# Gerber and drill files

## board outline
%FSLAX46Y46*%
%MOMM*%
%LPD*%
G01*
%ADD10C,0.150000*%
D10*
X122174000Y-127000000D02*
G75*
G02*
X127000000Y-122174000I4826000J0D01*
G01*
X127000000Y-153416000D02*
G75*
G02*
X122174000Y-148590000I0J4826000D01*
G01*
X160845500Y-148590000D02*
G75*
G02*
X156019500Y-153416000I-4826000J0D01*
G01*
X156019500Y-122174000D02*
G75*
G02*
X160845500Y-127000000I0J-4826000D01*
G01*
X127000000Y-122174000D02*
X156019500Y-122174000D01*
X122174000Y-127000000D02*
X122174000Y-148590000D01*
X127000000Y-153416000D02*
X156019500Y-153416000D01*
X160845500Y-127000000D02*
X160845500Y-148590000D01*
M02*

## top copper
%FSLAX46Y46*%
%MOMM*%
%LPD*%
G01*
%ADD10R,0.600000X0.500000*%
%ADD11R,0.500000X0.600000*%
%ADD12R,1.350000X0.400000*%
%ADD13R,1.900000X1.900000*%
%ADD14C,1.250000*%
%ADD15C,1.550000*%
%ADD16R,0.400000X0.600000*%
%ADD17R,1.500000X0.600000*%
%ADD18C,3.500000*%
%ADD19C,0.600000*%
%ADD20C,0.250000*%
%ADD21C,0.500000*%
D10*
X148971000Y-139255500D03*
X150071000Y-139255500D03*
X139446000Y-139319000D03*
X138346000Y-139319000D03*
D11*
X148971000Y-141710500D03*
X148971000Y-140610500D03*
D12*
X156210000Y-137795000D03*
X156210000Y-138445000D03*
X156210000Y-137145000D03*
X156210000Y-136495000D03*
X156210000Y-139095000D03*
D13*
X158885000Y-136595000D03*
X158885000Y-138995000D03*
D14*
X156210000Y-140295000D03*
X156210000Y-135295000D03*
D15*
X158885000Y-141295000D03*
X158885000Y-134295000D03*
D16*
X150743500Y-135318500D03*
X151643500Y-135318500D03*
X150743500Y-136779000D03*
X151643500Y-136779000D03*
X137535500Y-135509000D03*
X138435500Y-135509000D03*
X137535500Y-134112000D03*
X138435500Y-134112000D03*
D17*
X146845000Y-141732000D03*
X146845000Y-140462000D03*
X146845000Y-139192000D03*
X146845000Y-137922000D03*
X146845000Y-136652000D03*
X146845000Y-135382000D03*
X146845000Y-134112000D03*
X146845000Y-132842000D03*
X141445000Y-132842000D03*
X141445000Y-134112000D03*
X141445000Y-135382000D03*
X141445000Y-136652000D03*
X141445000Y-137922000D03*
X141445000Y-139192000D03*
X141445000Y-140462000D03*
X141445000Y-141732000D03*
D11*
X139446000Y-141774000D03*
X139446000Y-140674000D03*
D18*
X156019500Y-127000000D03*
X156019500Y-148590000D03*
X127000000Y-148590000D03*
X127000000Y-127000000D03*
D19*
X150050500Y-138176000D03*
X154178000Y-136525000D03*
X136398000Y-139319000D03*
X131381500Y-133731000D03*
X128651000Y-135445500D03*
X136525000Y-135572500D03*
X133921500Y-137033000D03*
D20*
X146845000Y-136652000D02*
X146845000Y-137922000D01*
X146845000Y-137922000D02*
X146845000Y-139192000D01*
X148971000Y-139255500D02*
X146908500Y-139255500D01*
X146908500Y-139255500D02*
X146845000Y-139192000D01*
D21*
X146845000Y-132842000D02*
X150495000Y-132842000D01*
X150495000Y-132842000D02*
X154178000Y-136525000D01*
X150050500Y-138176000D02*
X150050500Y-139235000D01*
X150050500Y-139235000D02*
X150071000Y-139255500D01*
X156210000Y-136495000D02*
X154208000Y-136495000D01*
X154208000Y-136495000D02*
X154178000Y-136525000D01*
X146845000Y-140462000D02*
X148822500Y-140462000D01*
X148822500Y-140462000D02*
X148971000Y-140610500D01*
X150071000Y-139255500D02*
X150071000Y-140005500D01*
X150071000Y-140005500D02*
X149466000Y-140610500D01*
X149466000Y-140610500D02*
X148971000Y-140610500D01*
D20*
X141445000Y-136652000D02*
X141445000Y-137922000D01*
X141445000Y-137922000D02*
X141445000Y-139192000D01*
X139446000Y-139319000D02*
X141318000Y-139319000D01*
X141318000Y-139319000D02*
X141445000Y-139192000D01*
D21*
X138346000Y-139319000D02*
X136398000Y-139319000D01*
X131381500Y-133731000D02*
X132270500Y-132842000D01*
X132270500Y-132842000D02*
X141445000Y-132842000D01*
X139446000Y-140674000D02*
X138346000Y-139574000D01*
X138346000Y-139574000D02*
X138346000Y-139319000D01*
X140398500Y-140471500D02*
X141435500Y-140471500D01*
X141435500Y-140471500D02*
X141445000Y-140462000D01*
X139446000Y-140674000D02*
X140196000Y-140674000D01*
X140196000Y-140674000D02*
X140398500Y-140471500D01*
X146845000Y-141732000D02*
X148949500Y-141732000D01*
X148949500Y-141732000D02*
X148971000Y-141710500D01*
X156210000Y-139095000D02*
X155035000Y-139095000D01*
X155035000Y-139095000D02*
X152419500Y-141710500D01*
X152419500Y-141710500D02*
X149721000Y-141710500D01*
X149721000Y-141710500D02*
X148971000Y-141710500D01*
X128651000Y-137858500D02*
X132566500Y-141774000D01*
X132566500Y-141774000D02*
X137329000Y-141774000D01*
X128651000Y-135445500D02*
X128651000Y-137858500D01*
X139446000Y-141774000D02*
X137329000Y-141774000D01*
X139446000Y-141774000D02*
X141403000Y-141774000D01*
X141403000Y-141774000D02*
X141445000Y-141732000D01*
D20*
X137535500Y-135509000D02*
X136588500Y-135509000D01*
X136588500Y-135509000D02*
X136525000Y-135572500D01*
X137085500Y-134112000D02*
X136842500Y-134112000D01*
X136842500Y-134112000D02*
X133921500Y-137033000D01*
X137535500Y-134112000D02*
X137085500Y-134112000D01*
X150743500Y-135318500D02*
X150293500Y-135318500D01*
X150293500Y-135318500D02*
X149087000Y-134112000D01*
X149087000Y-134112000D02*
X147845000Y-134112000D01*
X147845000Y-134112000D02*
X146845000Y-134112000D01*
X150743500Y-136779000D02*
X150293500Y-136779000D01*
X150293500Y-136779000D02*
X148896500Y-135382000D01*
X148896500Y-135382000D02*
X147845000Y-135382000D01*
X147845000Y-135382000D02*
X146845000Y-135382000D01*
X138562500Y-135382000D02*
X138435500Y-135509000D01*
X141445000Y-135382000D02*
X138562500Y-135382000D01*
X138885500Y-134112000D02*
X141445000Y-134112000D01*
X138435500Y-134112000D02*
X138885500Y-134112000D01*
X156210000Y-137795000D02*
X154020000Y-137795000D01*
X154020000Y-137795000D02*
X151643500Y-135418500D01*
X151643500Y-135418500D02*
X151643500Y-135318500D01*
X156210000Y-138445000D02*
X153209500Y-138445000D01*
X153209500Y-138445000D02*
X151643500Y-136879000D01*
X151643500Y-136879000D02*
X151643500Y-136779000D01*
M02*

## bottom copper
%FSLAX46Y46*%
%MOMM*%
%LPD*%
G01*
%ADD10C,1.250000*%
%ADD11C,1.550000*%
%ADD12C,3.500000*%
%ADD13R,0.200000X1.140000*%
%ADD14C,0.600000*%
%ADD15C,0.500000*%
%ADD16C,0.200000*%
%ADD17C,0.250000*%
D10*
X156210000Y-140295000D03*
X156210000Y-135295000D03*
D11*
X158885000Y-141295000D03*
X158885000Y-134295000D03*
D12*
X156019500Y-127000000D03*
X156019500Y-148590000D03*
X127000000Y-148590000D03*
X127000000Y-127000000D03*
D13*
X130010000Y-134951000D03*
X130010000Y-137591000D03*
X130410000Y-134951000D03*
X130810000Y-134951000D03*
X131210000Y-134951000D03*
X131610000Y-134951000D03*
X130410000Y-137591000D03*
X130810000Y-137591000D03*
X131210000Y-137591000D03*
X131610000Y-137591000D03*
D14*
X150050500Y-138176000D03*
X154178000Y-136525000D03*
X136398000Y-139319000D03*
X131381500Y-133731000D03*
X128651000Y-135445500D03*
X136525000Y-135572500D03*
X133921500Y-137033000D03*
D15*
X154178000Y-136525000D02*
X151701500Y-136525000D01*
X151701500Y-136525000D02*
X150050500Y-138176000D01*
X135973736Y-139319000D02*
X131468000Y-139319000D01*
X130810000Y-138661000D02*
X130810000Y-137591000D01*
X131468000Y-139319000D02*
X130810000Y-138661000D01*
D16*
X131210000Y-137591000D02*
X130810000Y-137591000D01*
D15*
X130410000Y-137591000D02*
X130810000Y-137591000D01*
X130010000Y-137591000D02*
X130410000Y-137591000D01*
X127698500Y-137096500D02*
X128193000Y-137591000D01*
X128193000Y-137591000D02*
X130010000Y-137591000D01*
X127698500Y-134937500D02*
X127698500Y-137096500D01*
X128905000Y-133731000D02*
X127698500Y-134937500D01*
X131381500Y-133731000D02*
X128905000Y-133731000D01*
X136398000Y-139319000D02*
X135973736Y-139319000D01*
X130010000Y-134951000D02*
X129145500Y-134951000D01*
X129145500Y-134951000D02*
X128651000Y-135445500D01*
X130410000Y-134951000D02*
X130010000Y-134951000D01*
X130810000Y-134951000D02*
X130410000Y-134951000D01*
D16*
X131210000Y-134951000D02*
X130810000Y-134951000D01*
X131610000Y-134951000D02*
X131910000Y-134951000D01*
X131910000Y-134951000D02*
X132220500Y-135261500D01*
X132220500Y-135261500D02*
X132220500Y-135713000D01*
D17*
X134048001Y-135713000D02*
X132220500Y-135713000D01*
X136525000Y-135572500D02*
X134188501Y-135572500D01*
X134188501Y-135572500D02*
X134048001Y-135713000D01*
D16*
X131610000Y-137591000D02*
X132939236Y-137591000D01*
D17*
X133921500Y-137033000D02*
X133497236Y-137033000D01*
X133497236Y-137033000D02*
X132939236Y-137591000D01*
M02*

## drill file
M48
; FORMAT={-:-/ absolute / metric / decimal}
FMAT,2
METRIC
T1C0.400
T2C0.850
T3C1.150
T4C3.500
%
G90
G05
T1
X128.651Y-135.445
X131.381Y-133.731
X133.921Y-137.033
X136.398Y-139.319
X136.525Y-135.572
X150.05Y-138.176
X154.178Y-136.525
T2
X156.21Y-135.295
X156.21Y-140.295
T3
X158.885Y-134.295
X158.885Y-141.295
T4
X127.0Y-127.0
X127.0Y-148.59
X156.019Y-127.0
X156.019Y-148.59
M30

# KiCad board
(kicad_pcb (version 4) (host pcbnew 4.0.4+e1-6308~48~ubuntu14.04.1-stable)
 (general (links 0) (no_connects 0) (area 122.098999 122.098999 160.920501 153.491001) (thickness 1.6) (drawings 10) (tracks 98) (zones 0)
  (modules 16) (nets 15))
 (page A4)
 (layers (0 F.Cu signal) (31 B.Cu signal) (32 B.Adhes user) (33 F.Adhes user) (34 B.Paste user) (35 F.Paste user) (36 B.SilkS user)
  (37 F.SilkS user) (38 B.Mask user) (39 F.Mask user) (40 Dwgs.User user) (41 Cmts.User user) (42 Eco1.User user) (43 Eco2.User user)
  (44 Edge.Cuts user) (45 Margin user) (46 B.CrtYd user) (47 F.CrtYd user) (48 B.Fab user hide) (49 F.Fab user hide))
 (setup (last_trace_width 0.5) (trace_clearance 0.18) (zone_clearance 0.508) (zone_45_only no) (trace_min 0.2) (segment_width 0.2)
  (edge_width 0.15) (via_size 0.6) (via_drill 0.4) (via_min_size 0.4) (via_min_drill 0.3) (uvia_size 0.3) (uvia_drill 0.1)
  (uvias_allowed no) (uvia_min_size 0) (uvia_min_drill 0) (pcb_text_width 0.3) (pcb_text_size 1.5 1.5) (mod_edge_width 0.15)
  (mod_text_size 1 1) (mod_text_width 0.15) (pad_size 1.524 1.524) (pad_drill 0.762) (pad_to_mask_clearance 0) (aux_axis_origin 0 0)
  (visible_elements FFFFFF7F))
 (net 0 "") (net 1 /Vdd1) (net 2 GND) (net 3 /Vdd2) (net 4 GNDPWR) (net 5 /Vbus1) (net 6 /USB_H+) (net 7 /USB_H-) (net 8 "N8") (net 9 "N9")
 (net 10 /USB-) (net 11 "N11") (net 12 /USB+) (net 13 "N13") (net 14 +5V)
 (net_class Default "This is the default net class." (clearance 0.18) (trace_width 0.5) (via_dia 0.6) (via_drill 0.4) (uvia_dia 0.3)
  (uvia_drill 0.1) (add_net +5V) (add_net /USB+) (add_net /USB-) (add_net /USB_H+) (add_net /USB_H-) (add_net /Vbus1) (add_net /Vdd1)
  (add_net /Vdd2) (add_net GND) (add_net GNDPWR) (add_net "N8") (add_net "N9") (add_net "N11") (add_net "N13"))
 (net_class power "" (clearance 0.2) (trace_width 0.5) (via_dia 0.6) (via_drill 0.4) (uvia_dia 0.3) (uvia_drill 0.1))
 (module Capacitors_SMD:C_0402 (layer F.Cu) (at 149.521 139.2555)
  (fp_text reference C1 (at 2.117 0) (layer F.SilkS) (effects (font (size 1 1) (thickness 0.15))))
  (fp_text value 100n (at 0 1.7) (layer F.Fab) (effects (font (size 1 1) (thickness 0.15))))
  (pad 1 smd rect (at -0.55 0) (size 0.6 0.5) (layers F.Cu F.Paste F.Mask) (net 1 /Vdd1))
  (pad 2 smd rect (at 0.55 0) (size 0.6 0.5) (layers F.Cu F.Paste F.Mask) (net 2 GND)))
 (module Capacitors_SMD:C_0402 (layer F.Cu) (at 138.896 139.319 180)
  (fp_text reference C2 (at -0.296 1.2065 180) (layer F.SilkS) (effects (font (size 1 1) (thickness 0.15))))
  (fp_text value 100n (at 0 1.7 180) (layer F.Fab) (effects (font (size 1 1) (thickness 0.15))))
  (pad 1 smd rect (at -0.55 0 180) (size 0.6 0.5) (layers F.Cu F.Paste F.Mask) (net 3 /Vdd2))
  (pad 2 smd rect (at 0.55 0 180) (size 0.6 0.5) (layers F.Cu F.Paste F.Mask) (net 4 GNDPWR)))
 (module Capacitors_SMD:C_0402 (layer F.Cu) (at 148.971 141.1605 90)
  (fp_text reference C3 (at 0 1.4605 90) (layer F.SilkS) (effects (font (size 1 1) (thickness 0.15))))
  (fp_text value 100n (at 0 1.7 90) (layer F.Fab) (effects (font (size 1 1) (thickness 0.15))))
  (pad 1 smd rect (at -0.55 0 90) (size 0.6 0.5) (layers F.Cu F.Paste F.Mask) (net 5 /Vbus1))
  (pad 2 smd rect (at 0.55 0 90) (size 0.6 0.5) (layers F.Cu F.Paste F.Mask) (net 2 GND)))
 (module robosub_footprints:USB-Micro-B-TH (layer F.Cu) (at 155.535 137.795 90)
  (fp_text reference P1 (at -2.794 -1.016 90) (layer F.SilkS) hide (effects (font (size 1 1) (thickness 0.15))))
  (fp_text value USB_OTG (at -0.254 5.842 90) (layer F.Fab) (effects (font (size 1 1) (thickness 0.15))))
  (pad 3 smd rect (at 0 0.675 90) (size 0.4 1.35) (layers F.Cu F.Paste F.Mask) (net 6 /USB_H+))
  (pad 2 smd rect (at -0.65 0.675 90) (size 0.4 1.35) (layers F.Cu F.Paste F.Mask) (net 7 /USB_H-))
  (pad 4 smd rect (at 0.65 0.675 90) (size 0.4 1.35) (layers F.Cu F.Paste F.Mask))
  (pad 5 smd rect (at 1.3 0.675 90) (size 0.4 1.35) (layers F.Cu F.Paste F.Mask) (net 2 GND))
  (pad 1 smd rect (at -1.3 0.675 90) (size 0.4 1.35) (layers F.Cu F.Paste F.Mask) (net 5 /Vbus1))
  (pad "" smd rect (at 1.2 3.35 90) (size 1.9 1.9) (layers F.Cu F.Paste F.Mask))
  (pad "" smd rect (at -1.2 3.35 90) (size 1.9 1.9) (layers F.Cu F.Paste F.Mask))
  (pad "" thru_hole circle (at -2.5 0.675 90) (size 1.25 1.25) (drill 0.85) (layers *.Cu *.Mask F.SilkS))
  (pad "" thru_hole circle (at 2.5 0.675 90) (size 1.25 1.25) (drill 0.85) (layers *.Cu *.Mask F.SilkS))
  (pad "" thru_hole circle (at -3.5 3.35 90) (size 1.55 1.55) (drill 1.15) (layers *.Cu *.Mask F.SilkS))
  (pad "" thru_hole circle (at 3.5 3.35 90) (size 1.55 1.55) (drill 1.15) (layers *.Cu *.Mask F.SilkS)))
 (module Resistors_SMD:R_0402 (layer F.Cu) (at 151.1935 135.3185)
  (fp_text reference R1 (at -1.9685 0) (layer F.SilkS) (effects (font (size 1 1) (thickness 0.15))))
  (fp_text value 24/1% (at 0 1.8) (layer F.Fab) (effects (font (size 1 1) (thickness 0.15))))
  (pad 1 smd rect (at -0.45 0) (size 0.4 0.6) (layers F.Cu F.Paste F.Mask) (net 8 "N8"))
  (pad 2 smd rect (at 0.45 0) (size 0.4 0.6) (layers F.Cu F.Paste F.Mask) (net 6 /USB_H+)))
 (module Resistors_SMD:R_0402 (layer F.Cu) (at 151.1935 136.779)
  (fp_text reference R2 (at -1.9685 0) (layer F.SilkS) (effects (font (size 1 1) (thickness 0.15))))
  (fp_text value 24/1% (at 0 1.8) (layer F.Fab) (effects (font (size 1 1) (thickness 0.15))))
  (pad 1 smd rect (at -0.45 0) (size 0.4 0.6) (layers F.Cu F.Paste F.Mask) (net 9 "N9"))
  (pad 2 smd rect (at 0.45 0) (size 0.4 0.6) (layers F.Cu F.Paste F.Mask) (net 7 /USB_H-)))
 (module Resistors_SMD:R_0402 (layer F.Cu) (at 137.9855 135.509)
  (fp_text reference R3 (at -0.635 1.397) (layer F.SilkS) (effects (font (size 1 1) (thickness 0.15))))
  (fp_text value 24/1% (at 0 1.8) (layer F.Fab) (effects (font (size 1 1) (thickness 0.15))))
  (pad 1 smd rect (at -0.45 0) (size 0.4 0.6) (layers F.Cu F.Paste F.Mask) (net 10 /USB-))
  (pad 2 smd rect (at 0.45 0) (size 0.4 0.6) (layers F.Cu F.Paste F.Mask) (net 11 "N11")))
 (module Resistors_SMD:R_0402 (layer F.Cu) (at 137.9855 134.112)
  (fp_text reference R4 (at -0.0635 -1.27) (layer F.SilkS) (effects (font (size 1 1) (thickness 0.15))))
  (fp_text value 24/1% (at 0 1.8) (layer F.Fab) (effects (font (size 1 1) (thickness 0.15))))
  (pad 1 smd rect (at -0.45 0) (size 0.4 0.6) (layers F.Cu F.Paste F.Mask) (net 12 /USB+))
  (pad 2 smd rect (at 0.45 0) (size 0.4 0.6) (layers F.Cu F.Paste F.Mask) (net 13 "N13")))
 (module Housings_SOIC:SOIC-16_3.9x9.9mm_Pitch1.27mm (layer F.Cu) (at 144.145 137.287 180)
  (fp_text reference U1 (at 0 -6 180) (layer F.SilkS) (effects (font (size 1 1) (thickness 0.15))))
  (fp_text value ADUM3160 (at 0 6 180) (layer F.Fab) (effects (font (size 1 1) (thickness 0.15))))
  (pad 1 smd rect (at -2.7 -4.445 180) (size 1.5 0.6) (layers F.Cu F.Paste F.Mask) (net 5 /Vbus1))
  (pad 2 smd rect (at -2.7 -3.175 180) (size 1.5 0.6) (layers F.Cu F.Paste F.Mask) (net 2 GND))
  (pad 3 smd rect (at -2.7 -1.905 180) (size 1.5 0.6) (layers F.Cu F.Paste F.Mask) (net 1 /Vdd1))
  (pad 4 smd rect (at -2.7 -0.635 180) (size 1.5 0.6) (layers F.Cu F.Paste F.Mask) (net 1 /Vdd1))
  (pad 5 smd rect (at -2.7 0.635 180) (size 1.5 0.6) (layers F.Cu F.Paste F.Mask) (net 1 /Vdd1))
  (pad 6 smd rect (at -2.7 1.905 180) (size 1.5 0.6) (layers F.Cu F.Paste F.Mask) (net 9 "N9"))
  (pad 7 smd rect (at -2.7 3.175 180) (size 1.5 0.6) (layers F.Cu F.Paste F.Mask) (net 8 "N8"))
  (pad 8 smd rect (at -2.7 4.445 180) (size 1.5 0.6) (layers F.Cu F.Paste F.Mask) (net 2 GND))
  (pad 9 smd rect (at 2.7 4.445 180) (size 1.5 0.6) (layers F.Cu F.Paste F.Mask) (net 4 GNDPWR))
  (pad 10 smd rect (at 2.7 3.175 180) (size 1.5 0.6) (layers F.Cu F.Paste F.Mask) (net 13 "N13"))
  (pad 11 smd rect (at 2.7 1.905 180) (size 1.5 0.6) (layers F.Cu F.Paste F.Mask) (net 11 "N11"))
  (pad 12 smd rect (at 2.7 0.635 180) (size 1.5 0.6) (layers F.Cu F.Paste F.Mask) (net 3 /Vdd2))
  (pad 13 smd rect (at 2.7 -0.635 180) (size 1.5 0.6) (layers F.Cu F.Paste F.Mask) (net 3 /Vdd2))
  (pad 14 smd rect (at 2.7 -1.905 180) (size 1.5 0.6) (layers F.Cu F.Paste F.Mask) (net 3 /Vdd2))
  (pad 15 smd rect (at 2.7 -3.175 180) (size 1.5 0.6) (layers F.Cu F.Paste F.Mask) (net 4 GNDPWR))
  (pad 16 smd rect (at 2.7 -4.445 180) (size 1.5 0.6) (layers F.Cu F.Paste F.Mask) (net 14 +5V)))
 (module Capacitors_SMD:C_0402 (layer F.Cu) (at 139.446 141.224 90)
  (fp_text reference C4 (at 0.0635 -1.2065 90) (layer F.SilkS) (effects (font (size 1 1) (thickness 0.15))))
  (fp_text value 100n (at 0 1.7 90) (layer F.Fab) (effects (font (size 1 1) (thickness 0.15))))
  (pad 1 smd rect (at -0.55 0 90) (size 0.6 0.5) (layers F.Cu F.Paste F.Mask) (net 14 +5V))
  (pad 2 smd rect (at 0.55 0 90) (size 0.6 0.5) (layers F.Cu F.Paste F.Mask) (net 4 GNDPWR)))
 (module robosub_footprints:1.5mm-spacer (layer F.Cu) (at 156.0195 127)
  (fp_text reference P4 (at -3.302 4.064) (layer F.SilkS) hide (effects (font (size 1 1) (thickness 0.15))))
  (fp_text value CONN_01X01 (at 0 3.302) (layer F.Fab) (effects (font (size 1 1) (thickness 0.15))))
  (pad "" thru_hole circle (at 0 0) (size 3.5 3.5) (drill 3.5) (layers *.Cu *.Mask F.SilkS)))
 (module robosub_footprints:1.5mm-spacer (layer F.Cu) (at 156.0195 148.59)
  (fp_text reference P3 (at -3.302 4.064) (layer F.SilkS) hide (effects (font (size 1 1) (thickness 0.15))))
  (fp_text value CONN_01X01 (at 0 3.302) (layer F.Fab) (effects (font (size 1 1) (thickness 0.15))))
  (pad "" thru_hole circle (at 0 0) (size 3.5 3.5) (drill 3.5) (layers *.Cu *.Mask F.SilkS)))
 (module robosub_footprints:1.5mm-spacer (layer F.Cu) (at 127 148.59)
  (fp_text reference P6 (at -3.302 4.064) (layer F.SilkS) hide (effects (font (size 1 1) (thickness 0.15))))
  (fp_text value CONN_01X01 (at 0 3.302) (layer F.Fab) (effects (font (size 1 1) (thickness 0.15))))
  (pad "" thru_hole circle (at 0 0) (size 3.5 3.5) (drill 3.5) (layers *.Cu *.Mask F.SilkS)))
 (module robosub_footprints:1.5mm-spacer (layer F.Cu) (at 127 127)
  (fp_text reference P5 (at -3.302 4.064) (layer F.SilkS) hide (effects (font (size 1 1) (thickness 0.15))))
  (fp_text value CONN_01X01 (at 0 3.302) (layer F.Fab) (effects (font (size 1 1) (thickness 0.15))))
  (pad "" thru_hole circle (at 0 0) (size 3.5 3.5) (drill 3.5) (layers *.Cu *.Mask F.SilkS)))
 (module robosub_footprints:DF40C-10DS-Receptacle (layer B.Cu) (at 130.81 136.271)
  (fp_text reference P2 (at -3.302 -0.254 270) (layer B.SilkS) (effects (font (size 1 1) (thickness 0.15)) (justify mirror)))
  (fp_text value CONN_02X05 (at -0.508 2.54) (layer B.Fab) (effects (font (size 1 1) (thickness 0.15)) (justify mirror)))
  (pad 1 smd rect (at -0.8 -1.32 270) (size 1.14 0.2) (layers B.Cu B.Paste B.Mask) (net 14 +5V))
  (pad 2 smd rect (at -0.8 1.32 270) (size 1.14 0.2) (layers B.Cu B.Paste B.Mask) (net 4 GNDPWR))
  (pad 3 smd rect (at -0.4 -1.32 270) (size 1.14 0.2) (layers B.Cu B.Paste B.Mask) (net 14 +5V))
  (pad 5 smd rect (at 0 -1.32 270) (size 1.14 0.2) (layers B.Cu B.Paste B.Mask) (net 14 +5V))
  (pad 7 smd rect (at 0.4 -1.32 270) (size 1.14 0.2) (layers B.Cu B.Paste B.Mask) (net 14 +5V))
  (pad 9 smd rect (at 0.8 -1.32 270) (size 1.14 0.2) (layers B.Cu B.Paste B.Mask) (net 10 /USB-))
  (pad 4 smd rect (at -0.4 1.32 270) (size 1.14 0.2) (layers B.Cu B.Paste B.Mask) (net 4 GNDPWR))
  (pad 6 smd rect (at 0 1.32 270) (size 1.14 0.2) (layers B.Cu B.Paste B.Mask) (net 4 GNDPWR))
  (pad 8 smd rect (at 0.4 1.32 270) (size 1.14 0.2) (layers B.Cu B.Paste B.Mask) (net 4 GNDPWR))
  (pad 10 smd rect (at 0.8 1.32 270) (size 1.14 0.2) (layers B.Cu B.Paste B.Mask) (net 12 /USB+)))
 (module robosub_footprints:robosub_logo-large (layer F.Cu) (at 141.6685 148.59)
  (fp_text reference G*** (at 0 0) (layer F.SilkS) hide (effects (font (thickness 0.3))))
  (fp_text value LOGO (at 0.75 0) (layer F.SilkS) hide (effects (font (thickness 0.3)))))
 (gr_arc (start 127 127) (end 122.174 127) (angle 90) (layer Edge.Cuts) (width 0.15))
 (gr_arc (start 127 148.59) (end 127 153.416) (angle 90) (layer Edge.Cuts) (width 0.15))
 (gr_arc (start 156.0195 148.59) (end 160.8455 148.59) (angle 90) (layer Edge.Cuts) (width 0.15))
 (gr_arc (start 156.0195 127) (end 156.0195 122.174) (angle 90) (layer Edge.Cuts) (width 0.15))
 (gr_line (start 127 122.174) (end 156.0195 122.174) (layer Edge.Cuts) (width 0.15))
 (gr_line (start 122.174 127) (end 122.174 148.59) (layer Edge.Cuts) (width 0.15))
 (gr_line (start 127 153.416) (end 156.0195 153.416) (layer Edge.Cuts) (width 0.15))
 (gr_line (start 160.8455 127) (end 160.8455 148.59) (layer Edge.Cuts) (width 0.15))
 (segment (start 146.845 136.652) (end 146.845 137.922) (width 0.25) (layer F.Cu) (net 1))
 (segment (start 146.845 137.922) (end 146.845 139.192) (width 0.25) (layer F.Cu) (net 1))
 (segment (start 148.971 139.2555) (end 146.9085 139.2555) (width 0.25) (layer F.Cu) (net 1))
 (segment (start 146.9085 139.2555) (end 146.845 139.192) (width 0.25) (layer F.Cu) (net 1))
 (segment (start 146.845 132.842) (end 150.495 132.842) (width 0.5) (layer F.Cu) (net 2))
 (segment (start 150.495 132.842) (end 154.178 136.525) (width 0.5) (layer F.Cu) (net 2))
 (segment (start 150.0505 138.176) (end 150.0505 139.235) (width 0.5) (layer F.Cu) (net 2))
 (segment (start 150.0505 139.235) (end 150.071 139.2555) (width 0.5) (layer F.Cu) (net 2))
 (segment (start 154.178 136.525) (end 151.7015 136.525) (width 0.5) (layer B.Cu) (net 2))
 (segment (start 151.7015 136.525) (end 150.0505 138.176) (width 0.5) (layer B.Cu) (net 2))
 (via (at 150.0505 138.176) (size 0.6) (drill 0.4) (layers F.Cu B.Cu) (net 2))
 (segment (start 156.21 136.495) (end 154.208 136.495) (width 0.5) (layer F.Cu) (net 2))
 (segment (start 154.208 136.495) (end 154.178 136.525) (width 0.5) (layer F.Cu) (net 2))
 (via (at 154.178 136.525) (size 0.6) (drill 0.4) (layers F.Cu B.Cu) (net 2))
 (segment (start 146.845 140.462) (end 148.8225 140.462) (width 0.5) (layer F.Cu) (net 2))
 (segment (start 148.8225 140.462) (end 148.971 140.6105) (width 0.5) (layer F.Cu) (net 2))
 (segment (start 150.071 139.2555) (end 150.071 140.0055) (width 0.5) (layer F.Cu) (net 2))
 (segment (start 150.071 140.0055) (end 149.466 140.6105) (width 0.5) (layer F.Cu) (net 2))
 (segment (start 149.466 140.6105) (end 148.971 140.6105) (width 0.5) (layer F.Cu) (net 2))
 (segment (start 141.445 136.652) (end 141.445 137.922) (width 0.25) (layer F.Cu) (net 3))
 (segment (start 141.445 137.922) (end 141.445 139.192) (width 0.25) (layer F.Cu) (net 3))
 (segment (start 139.446 139.319) (end 141.318 139.319) (width 0.25) (layer F.Cu) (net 3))
 (segment (start 141.318 139.319) (end 141.445 139.192) (width 0.25) (layer F.Cu) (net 3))
 (segment (start 135.973736 139.319) (end 131.468 139.319) (width 0.5) (layer B.Cu) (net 4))
 (segment (start 130.81 138.661) (end 130.81 137.591) (width 0.5) (layer B.Cu) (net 4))
 (segment (start 131.468 139.319) (end 130.81 138.661) (width 0.5) (layer B.Cu) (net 4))
 (segment (start 131.21 137.591) (end 130.81 137.591) (width 0.2) (layer B.Cu) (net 4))
 (segment (start 130.41 137.591) (end 130.81 137.591) (width 0.5) (layer B.Cu) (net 4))
 (segment (start 130.01 137.591) (end 130.41 137.591) (width 0.5) (layer B.Cu) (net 4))
 (segment (start 127.6985 137.0965) (end 128.193 137.591) (width 0.5) (layer B.Cu) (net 4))
 (segment (start 128.193 137.591) (end 130.01 137.591) (width 0.5) (layer B.Cu) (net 4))
 (segment (start 127.6985 134.9375) (end 127.6985 137.0965) (width 0.5) (layer B.Cu) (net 4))
 (segment (start 128.905 133.731) (end 127.6985 134.9375) (width 0.5) (layer B.Cu) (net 4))
 (segment (start 131.3815 133.731) (end 128.905 133.731) (width 0.5) (layer B.Cu) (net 4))
 (segment (start 136.398 139.319) (end 135.973736 139.319) (width 0.5) (layer B.Cu) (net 4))
 (via (at 136.398 139.319) (size 0.6) (drill 0.4) (layers F.Cu B.Cu) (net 4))
 (segment (start 138.346 139.319) (end 136.398 139.319) (width 0.5) (layer F.Cu) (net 4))
 (segment (start 131.3815 133.731) (end 132.2705 132.842) (width 0.5) (layer F.Cu) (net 4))
 (segment (start 132.2705 132.842) (end 141.445 132.842) (width 0.5) (layer F.Cu) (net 4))
 (via (at 131.3815 133.731) (size 0.6) (drill 0.4) (layers F.Cu B.Cu) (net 4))
 (segment (start 139.446 140.674) (end 138.346 139.574) (width 0.5) (layer F.Cu) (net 4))
 (segment (start 138.346 139.574) (end 138.346 139.319) (width 0.5) (layer F.Cu) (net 4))
 (segment (start 140.3985 140.4715) (end 141.4355 140.4715) (width 0.5) (layer F.Cu) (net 4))
 (segment (start 141.4355 140.4715) (end 141.445 140.462) (width 0.5) (layer F.Cu) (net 4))
 (segment (start 139.446 140.674) (end 140.196 140.674) (width 0.5) (layer F.Cu) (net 4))
 (segment (start 140.196 140.674) (end 140.3985 140.4715) (width 0.5) (layer F.Cu) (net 4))
 (segment (start 146.845 141.732) (end 148.9495 141.732) (width 0.5) (layer F.Cu) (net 5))
 (segment (start 148.9495 141.732) (end 148.971 141.7105) (width 0.5) (layer F.Cu) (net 5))
 (segment (start 156.21 139.095) (end 155.035 139.095) (width 0.5) (layer F.Cu) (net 5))
 (segment (start 155.035 139.095) (end 152.4195 141.7105) (width 0.5) (layer F.Cu) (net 5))
 (segment (start 152.4195 141.7105) (end 149.721 141.7105) (width 0.5) (layer F.Cu) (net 5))
 (segment (start 149.721 141.7105) (end 148.971 141.7105) (width 0.5) (layer F.Cu) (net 5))
 (segment (start 128.651 137.8585) (end 132.5665 141.774) (width 0.5) (layer F.Cu) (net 14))
 (segment (start 132.5665 141.774) (end 137.329 141.774) (width 0.5) (layer F.Cu) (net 14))
 (segment (start 128.651 135.4455) (end 128.651 137.8585) (width 0.5) (layer F.Cu) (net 14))
 (segment (start 130.01 134.951) (end 129.1455 134.951) (width 0.5) (layer B.Cu) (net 14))
 (segment (start 129.1455 134.951) (end 128.651 135.4455) (width 0.5) (layer B.Cu) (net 14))
 (via (at 128.651 135.4455) (size 0.6) (drill 0.4) (layers F.Cu B.Cu) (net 14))
 (segment (start 130.41 134.951) (end 130.01 134.951) (width 0.5) (layer B.Cu) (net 14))
 (segment (start 130.81 134.951) (end 130.41 134.951) (width 0.5) (layer B.Cu) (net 14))
 (segment (start 131.21 134.951) (end 130.81 134.951) (width 0.2) (layer B.Cu) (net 14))
 (segment (start 139.446 141.774) (end 137.329 141.774) (width 0.5) (layer F.Cu) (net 14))
 (segment (start 139.446 141.774) (end 141.403 141.774) (width 0.5) (layer F.Cu) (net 14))
 (segment (start 141.403 141.774) (end 141.445 141.732) (width 0.5) (layer F.Cu) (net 14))
 (segment (start 131.61 134.951) (end 131.91 134.951) (width 0.2) (layer B.Cu) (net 10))
 (segment (start 131.91 134.951) (end 132.2205 135.2615) (width 0.2) (layer B.Cu) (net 10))
 (segment (start 132.2205 135.2615) (end 132.2205 135.713) (width 0.2) (layer B.Cu) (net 10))
 (segment (start 134.048001 135.713) (end 132.2205 135.713) (width 0.25) (layer B.Cu) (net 10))
 (segment (start 136.525 135.5725) (end 134.188501 135.5725) (width 0.25) (layer B.Cu) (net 10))
 (segment (start 134.188501 135.5725) (end 134.048001 135.713) (width 0.25) (layer B.Cu) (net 10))
 (via (at 136.525 135.5725) (size 0.6) (drill 0.4) (layers F.Cu B.Cu) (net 10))
 (segment (start 137.5355 135.509) (end 136.5885 135.509) (width 0.25) (layer F.Cu) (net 10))
 (segment (start 136.5885 135.509) (end 136.525 135.5725) (width 0.25) (layer F.Cu) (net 10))
 (segment (start 131.61 137.591) (end 132.939236 137.591) (width 0.2) (layer B.Cu) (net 12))
 (segment (start 133.9215 137.033) (end 133.497236 137.033) (width 0.25) (layer B.Cu) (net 12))
 (segment (start 133.497236 137.033) (end 132.939236 137.591) (width 0.25) (layer B.Cu) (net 12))
 (segment (start 137.0855 134.112) (end 136.8425 134.112) (width 0.25) (layer F.Cu) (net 12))
 (segment (start 136.8425 134.112) (end 133.9215 137.033) (width 0.25) (layer F.Cu) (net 12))
 (via (at 133.9215 137.033) (size 0.6) (drill 0.4) (layers F.Cu B.Cu) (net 12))
 (segment (start 137.5355 134.112) (end 137.0855 134.112) (width 0.25) (layer F.Cu) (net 12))
 (segment (start 150.7435 135.3185) (end 150.2935 135.3185) (width 0.25) (layer F.Cu) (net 8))
 (segment (start 150.2935 135.3185) (end 149.087 134.112) (width 0.25) (layer F.Cu) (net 8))
 (segment (start 149.087 134.112) (end 147.845 134.112) (width 0.25) (layer F.Cu) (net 8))
 (segment (start 147.845 134.112) (end 146.845 134.112) (width 0.25) (layer F.Cu) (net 8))
 (segment (start 150.7435 136.779) (end 150.2935 136.779) (width 0.25) (layer F.Cu) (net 9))
 (segment (start 150.2935 136.779) (end 148.8965 135.382) (width 0.25) (layer F.Cu) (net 9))
 (segment (start 148.8965 135.382) (end 147.845 135.382) (width 0.25) (layer F.Cu) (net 9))
 (segment (start 147.845 135.382) (end 146.845 135.382) (width 0.25) (layer F.Cu) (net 9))
 (segment (start 138.5625 135.382) (end 138.4355 135.509) (width 0.25) (layer F.Cu) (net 11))
 (segment (start 141.445 135.382) (end 138.5625 135.382) (width 0.25) (layer F.Cu) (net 11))
 (segment (start 138.8855 134.112) (end 141.445 134.112) (width 0.25) (layer F.Cu) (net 13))
 (segment (start 138.4355 134.112) (end 138.8855 134.112) (width 0.25) (layer F.Cu) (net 13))
 (segment (start 156.21 137.795) (end 154.02 137.795) (width 0.25) (layer F.Cu) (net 6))
 (segment (start 154.02 137.795) (end 151.6435 135.4185) (width 0.25) (layer F.Cu) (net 6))
 (segment (start 151.6435 135.4185) (end 151.6435 135.3185) (width 0.25) (layer F.Cu) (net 6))
 (segment (start 156.21 138.445) (end 153.2095 138.445) (width 0.25) (layer F.Cu) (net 7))
 (segment (start 153.2095 138.445) (end 151.6435 136.879) (width 0.25) (layer F.Cu) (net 7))
 (segment (start 151.6435 136.879) (end 151.6435 136.779) (width 0.25) (layer F.Cu) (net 7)))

